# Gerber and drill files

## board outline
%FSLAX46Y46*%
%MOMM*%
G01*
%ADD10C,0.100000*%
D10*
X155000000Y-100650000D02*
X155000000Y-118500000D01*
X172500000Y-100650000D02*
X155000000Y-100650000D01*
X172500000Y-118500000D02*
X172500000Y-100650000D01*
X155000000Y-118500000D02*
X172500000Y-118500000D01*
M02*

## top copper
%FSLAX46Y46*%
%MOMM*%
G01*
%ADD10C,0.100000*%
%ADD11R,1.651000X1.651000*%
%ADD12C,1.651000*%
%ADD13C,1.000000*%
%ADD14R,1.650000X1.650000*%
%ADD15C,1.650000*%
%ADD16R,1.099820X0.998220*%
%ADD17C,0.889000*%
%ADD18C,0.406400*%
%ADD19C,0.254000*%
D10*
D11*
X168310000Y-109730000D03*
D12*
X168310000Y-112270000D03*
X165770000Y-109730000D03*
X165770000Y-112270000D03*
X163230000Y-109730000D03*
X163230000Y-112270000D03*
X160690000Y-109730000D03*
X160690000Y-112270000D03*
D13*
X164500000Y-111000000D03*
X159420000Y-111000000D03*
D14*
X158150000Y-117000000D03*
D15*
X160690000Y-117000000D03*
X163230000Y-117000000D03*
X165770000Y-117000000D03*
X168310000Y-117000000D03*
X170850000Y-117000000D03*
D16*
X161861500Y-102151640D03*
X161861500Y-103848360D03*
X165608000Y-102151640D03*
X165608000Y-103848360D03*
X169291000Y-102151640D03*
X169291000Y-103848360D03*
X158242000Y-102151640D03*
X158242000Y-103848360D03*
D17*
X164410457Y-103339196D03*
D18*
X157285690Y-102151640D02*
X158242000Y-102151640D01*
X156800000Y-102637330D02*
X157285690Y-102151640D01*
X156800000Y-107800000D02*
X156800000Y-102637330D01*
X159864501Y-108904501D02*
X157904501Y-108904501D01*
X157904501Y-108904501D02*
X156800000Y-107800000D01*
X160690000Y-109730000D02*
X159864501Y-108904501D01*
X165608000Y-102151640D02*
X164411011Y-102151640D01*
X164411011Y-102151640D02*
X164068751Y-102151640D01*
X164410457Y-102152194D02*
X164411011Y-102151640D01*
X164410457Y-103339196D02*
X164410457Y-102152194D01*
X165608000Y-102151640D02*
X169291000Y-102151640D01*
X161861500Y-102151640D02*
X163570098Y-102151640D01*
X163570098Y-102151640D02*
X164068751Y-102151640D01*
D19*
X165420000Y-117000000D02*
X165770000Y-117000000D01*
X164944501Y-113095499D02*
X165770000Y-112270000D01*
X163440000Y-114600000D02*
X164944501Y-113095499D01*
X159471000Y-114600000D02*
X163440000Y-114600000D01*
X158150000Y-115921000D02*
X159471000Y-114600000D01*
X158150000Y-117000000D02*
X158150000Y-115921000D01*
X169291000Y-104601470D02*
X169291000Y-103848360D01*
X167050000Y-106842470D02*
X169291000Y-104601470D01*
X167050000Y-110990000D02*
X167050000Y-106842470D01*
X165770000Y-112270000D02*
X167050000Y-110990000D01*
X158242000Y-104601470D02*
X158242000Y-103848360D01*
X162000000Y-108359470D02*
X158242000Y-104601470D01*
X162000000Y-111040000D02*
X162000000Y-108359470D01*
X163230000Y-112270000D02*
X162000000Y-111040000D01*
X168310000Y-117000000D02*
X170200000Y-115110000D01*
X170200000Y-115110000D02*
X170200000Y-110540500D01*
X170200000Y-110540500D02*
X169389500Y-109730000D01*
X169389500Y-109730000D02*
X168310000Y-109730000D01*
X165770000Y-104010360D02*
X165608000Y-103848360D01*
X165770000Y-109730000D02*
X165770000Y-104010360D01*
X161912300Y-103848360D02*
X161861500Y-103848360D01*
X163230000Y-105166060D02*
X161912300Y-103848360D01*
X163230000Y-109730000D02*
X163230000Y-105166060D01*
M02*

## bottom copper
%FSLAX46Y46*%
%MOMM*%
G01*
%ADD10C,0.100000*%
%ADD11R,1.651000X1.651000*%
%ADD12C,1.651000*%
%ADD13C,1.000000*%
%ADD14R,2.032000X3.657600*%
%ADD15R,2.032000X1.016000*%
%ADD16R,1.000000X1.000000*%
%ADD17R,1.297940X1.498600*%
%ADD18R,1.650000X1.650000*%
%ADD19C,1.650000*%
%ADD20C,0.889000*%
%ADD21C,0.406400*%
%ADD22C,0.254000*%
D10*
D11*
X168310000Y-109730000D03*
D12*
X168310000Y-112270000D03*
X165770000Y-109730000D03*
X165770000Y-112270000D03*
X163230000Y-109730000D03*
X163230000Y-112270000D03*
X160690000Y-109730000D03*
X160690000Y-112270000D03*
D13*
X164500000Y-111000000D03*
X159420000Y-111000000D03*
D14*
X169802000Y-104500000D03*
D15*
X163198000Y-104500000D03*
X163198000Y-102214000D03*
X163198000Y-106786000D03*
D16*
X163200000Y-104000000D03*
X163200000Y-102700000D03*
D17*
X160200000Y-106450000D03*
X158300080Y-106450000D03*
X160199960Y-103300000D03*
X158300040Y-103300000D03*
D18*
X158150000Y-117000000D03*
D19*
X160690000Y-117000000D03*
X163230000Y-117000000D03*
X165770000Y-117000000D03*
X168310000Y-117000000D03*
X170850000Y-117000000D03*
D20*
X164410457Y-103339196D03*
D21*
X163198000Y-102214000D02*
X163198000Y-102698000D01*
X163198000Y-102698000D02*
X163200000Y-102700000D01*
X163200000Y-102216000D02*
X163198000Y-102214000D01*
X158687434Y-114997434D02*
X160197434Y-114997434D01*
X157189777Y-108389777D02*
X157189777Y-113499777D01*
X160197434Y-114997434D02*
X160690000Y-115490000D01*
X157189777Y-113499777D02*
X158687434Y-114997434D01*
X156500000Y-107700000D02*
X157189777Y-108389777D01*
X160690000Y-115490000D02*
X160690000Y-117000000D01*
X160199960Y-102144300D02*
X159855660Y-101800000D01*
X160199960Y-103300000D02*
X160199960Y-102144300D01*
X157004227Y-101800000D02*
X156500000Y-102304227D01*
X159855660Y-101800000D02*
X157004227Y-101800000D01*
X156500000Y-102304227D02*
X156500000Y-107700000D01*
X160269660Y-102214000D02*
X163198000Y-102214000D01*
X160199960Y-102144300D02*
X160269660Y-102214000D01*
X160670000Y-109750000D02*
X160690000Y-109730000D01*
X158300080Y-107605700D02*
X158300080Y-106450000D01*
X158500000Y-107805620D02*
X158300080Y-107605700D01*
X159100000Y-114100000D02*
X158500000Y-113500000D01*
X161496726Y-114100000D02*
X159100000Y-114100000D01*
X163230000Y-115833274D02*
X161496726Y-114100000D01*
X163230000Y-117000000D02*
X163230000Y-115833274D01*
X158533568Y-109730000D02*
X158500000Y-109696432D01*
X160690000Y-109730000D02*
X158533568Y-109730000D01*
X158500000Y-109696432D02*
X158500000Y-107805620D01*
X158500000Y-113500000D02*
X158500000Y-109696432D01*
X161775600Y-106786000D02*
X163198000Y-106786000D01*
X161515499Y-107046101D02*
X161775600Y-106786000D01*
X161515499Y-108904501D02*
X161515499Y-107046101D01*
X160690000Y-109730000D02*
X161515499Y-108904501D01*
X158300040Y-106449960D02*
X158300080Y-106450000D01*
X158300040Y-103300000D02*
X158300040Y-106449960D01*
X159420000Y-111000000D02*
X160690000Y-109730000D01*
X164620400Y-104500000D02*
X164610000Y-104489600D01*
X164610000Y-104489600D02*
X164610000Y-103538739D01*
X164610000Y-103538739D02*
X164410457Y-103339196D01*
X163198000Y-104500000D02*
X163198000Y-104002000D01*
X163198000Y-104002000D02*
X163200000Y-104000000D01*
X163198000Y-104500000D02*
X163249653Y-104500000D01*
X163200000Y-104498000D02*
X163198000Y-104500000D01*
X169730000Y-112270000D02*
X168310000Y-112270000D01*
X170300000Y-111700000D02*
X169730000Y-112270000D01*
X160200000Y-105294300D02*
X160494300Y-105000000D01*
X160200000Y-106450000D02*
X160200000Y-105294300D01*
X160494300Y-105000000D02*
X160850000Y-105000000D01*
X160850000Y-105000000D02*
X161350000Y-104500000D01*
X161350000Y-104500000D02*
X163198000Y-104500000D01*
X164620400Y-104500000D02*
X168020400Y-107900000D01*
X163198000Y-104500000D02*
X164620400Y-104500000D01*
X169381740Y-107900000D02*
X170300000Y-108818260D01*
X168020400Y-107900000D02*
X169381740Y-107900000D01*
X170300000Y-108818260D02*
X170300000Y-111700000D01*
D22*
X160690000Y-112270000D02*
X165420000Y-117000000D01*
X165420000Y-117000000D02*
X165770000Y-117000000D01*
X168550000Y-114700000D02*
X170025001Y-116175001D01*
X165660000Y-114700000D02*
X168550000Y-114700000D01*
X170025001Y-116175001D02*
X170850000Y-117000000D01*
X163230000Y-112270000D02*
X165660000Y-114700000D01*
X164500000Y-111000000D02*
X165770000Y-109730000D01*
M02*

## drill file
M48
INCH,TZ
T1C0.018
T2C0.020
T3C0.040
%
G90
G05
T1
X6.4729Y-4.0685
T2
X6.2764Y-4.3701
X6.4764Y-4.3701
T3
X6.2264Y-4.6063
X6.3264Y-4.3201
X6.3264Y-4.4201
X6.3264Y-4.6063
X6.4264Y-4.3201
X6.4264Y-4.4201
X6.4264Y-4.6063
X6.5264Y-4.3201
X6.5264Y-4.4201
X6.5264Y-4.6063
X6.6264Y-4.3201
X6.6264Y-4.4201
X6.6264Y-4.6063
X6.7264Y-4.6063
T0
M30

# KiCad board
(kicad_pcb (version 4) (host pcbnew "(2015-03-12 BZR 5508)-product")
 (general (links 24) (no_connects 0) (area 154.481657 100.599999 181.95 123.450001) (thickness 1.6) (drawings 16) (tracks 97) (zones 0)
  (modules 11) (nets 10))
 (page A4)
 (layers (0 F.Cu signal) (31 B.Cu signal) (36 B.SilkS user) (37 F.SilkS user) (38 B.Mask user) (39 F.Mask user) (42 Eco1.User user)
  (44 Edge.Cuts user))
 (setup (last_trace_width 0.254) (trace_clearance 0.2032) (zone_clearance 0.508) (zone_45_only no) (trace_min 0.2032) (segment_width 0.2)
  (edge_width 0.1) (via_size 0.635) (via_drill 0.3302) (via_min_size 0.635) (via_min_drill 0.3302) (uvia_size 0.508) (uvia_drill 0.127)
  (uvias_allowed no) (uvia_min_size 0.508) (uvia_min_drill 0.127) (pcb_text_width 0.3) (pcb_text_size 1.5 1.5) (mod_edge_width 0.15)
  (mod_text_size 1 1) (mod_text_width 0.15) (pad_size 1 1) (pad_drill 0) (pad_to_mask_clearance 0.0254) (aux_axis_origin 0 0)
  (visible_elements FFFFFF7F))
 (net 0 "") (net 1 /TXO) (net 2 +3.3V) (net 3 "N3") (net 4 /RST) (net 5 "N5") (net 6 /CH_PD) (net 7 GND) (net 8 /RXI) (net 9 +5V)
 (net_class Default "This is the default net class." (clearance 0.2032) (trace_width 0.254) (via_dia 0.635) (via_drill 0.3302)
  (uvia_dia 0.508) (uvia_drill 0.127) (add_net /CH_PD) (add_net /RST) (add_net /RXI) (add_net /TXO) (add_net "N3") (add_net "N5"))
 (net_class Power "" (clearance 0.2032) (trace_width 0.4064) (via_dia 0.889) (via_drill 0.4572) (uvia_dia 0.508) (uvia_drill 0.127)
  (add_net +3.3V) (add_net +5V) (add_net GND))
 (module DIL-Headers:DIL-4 (layer F.Cu) (at 164.5 111)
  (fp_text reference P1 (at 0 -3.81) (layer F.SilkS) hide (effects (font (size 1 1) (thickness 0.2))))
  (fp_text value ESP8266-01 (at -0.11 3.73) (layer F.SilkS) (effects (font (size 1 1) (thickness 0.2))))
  (pad 1 thru_hole rect (at 3.81 -1.27) (size 1.651 1.651) (drill 1.016) (layers *.Cu *.Mask F.SilkS) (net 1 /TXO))
  (pad 2 thru_hole circle (at 3.81 1.27) (size 1.651 1.651) (drill 1.016) (layers *.Cu *.Mask F.SilkS) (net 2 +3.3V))
  (pad 3 thru_hole circle (at 1.27 -1.27) (size 1.651 1.651) (drill 1.016) (layers *.Cu *.Mask F.SilkS) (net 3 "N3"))
  (pad 4 thru_hole circle (at 1.27 1.27) (size 1.651 1.651) (drill 1.016) (layers *.Cu *.Mask F.SilkS) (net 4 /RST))
  (pad 5 thru_hole circle (at -1.27 -1.27) (size 1.651 1.651) (drill 1.016) (layers *.Cu *.Mask F.SilkS) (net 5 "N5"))
  (pad 6 thru_hole circle (at -1.27 1.27) (size 1.651 1.651) (drill 1.016) (layers *.Cu *.Mask F.SilkS) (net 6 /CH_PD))
  (pad 7 thru_hole circle (at -3.81 -1.27) (size 1.651 1.651) (drill 1.016) (layers *.Cu *.Mask F.SilkS) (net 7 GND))
  (pad 8 thru_hole circle (at -3.81 1.27) (size 1.651 1.651) (drill 1.016) (layers *.Cu *.Mask F.SilkS) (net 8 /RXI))
  (pad 3 thru_hole circle (at 0 0) (size 1 1) (drill 0.5) (layers *.Cu *.Mask F.SilkS) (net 3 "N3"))
  (pad 7 thru_hole circle (at -5.08 0) (size 1 1) (drill 0.5) (layers *.Cu *.Mask F.SilkS) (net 7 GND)))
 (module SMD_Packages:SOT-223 (layer B.Cu) (at 166.5 104.5 90)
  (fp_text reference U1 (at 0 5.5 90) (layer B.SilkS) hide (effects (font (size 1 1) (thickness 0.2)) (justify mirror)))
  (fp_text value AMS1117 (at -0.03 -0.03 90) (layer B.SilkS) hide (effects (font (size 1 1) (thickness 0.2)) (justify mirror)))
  (pad 4 smd rect (at 0 3.302 90) (size 3.6576 2.032) (layers B.Cu B.Mask))
  (pad 2 smd rect (at 0 -3.302 90) (size 1.016 2.032) (layers B.Cu B.Mask) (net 2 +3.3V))
  (pad 3 smd rect (at 2.286 -3.302 90) (size 1.016 2.032) (layers B.Cu B.Mask) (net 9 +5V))
  (pad 1 smd rect (at -2.286 -3.302 90) (size 1.016 2.032) (layers B.Cu B.Mask) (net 7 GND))
  (pad 2 smd rect (at 0.5 -3.3 90) (size 1 1) (layers B.Cu B.Mask) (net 2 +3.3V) (solder_mask_margin 0.15) (clearance 0.01))
  (pad 3 smd rect (at 1.8 -3.3 90) (size 1 1) (layers B.Cu B.Mask) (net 9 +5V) (solder_mask_margin 0.15) (clearance 0.01)))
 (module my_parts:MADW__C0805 (layer B.Cu) (at 159.25004 106.45 180)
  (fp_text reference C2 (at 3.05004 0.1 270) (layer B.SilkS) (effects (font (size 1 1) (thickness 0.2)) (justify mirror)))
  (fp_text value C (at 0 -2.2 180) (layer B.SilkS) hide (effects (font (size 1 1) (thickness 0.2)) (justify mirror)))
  (pad 1 smd rect (at -0.94996 0 180) (size 1.29794 1.4986) (layers B.Cu B.Mask) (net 2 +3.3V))
  (pad 2 smd rect (at 0.94996 0 180) (size 1.29794 1.4986) (layers B.Cu B.Mask) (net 7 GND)))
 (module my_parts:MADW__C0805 (layer B.Cu) (at 159.25 103.3 180)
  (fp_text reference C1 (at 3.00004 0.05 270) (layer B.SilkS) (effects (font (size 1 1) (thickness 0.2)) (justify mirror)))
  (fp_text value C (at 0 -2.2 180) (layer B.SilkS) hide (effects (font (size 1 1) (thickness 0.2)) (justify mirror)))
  (pad 1 smd rect (at -0.94996 0 180) (size 1.29794 1.4986) (layers B.Cu B.Mask) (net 9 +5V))
  (pad 2 smd rect (at 0.94996 0 180) (size 1.29794 1.4986) (layers B.Cu B.Mask) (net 7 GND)))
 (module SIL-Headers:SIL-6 (layer F.Cu) (at 164.5 117)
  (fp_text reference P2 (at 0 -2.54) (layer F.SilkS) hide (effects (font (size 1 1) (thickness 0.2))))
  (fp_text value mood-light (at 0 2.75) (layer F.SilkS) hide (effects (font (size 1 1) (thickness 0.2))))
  (pad 1 thru_hole rect (at -6.35 0) (size 1.65 1.65) (drill 1.016) (layers *.Cu *.Mask F.SilkS) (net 4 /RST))
  (pad 2 thru_hole circle (at -3.81 0) (size 1.65 1.65) (drill 1.016) (layers *.Cu *.Mask F.SilkS) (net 9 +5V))
  (pad 3 thru_hole circle (at -1.27 0) (size 1.65 1.65) (drill 1.016) (layers *.Cu *.Mask F.SilkS) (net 7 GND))
  (pad 4 thru_hole circle (at 1.27 0) (size 1.65 1.65) (drill 1.016) (layers *.Cu *.Mask F.SilkS) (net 8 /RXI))
  (pad 5 thru_hole circle (at 3.81 0) (size 1.65 1.65) (drill 1.016) (layers *.Cu *.Mask F.SilkS) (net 1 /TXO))
  (pad 6 thru_hole circle (at 6.35 0) (size 1.65 1.65) (drill 1.016) (layers *.Cu *.Mask F.SilkS) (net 6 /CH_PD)))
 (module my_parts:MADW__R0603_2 (layer F.Cu) (at 161.8615 103 270)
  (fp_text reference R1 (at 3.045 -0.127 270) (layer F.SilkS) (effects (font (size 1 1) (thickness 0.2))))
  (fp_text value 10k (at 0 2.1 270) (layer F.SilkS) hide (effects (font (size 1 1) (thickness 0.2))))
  (pad 1 smd rect (at -0.84836 0 270) (size 0.99822 1.09982) (layers F.Cu F.Mask) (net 2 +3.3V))
  (pad 2 smd rect (at 0.84836 0 270) (size 0.99822 1.09982) (layers F.Cu F.Mask) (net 5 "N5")))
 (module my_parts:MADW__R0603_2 (layer F.Cu) (at 165.608 103 270)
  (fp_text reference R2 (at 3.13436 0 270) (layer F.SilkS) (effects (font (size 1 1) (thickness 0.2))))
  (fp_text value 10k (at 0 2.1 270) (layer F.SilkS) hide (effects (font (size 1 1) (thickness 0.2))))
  (pad 1 smd rect (at -0.84836 0 270) (size 0.99822 1.09982) (layers F.Cu F.Mask) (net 2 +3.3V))
  (pad 2 smd rect (at 0.84836 0 270) (size 0.99822 1.09982) (layers F.Cu F.Mask) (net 3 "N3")))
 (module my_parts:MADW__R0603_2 (layer F.Cu) (at 169.291 103 270)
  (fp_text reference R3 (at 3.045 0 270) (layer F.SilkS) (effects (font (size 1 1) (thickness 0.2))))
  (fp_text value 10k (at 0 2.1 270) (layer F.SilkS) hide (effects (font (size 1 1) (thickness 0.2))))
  (pad 1 smd rect (at -0.84836 0 270) (size 0.99822 1.09982) (layers F.Cu F.Mask) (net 2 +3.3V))
  (pad 2 smd rect (at 0.84836 0 270) (size 0.99822 1.09982) (layers F.Cu F.Mask) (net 4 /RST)))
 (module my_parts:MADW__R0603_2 (layer F.Cu) (at 158.242 103 270)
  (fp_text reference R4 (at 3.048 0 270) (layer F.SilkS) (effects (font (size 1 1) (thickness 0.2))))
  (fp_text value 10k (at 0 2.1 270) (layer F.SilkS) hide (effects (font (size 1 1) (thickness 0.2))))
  (pad 1 smd rect (at -0.84836 0 270) (size 0.99822 1.09982) (layers F.Cu F.Mask) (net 7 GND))
  (pad 2 smd rect (at 0.84836 0 270) (size 0.99822 1.09982) (layers F.Cu F.Mask) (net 6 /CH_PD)))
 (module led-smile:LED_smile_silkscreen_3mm (layer F.Cu) (at 157.05 109.75)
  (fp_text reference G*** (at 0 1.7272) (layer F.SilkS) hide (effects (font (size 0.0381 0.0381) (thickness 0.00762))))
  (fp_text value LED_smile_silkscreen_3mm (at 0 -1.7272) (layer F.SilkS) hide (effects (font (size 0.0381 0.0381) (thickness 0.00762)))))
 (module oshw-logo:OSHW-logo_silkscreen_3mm (layer F.Cu) (at 157 113)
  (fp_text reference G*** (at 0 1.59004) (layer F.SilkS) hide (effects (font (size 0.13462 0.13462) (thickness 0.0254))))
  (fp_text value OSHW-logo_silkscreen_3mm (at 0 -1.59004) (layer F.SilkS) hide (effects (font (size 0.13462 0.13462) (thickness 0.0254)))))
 (gr_line (start 155 100.65) (end 155 118.5) (layer Edge.Cuts) (width 0.1))
 (gr_line (start 172.5 100.65) (end 155 100.65) (layer Edge.Cuts) (width 0.1))
 (gr_line (start 172.5 118.5) (end 172.5 100.65) (layer Edge.Cuts) (width 0.1))
 (gr_line (start 155 118.5) (end 172.5 118.5) (layer Edge.Cuts) (width 0.1))
 (segment (start 163.198 102.214) (end 163.198 102.698) (width 0.4064) (layer B.Cu) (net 9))
 (segment (start 163.198 102.698) (end 163.2 102.7) (width 0.4064) (layer B.Cu) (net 9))
 (segment (start 163.2 102.216) (end 163.198 102.214) (width 0.4064) (layer B.Cu) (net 9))
 (segment (start 158.687434 114.997434) (end 160.197434 114.997434) (width 0.4064) (layer B.Cu) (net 9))
 (segment (start 157.189777 108.389777) (end 157.189777 113.499777) (width 0.4064) (layer B.Cu) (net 9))
 (segment (start 160.197434 114.997434) (end 160.69 115.49) (width 0.4064) (layer B.Cu) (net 9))
 (segment (start 157.189777 113.499777) (end 158.687434 114.997434) (width 0.4064) (layer B.Cu) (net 9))
 (segment (start 156.5 107.7) (end 157.189777 108.389777) (width 0.4064) (layer B.Cu) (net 9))
 (segment (start 160.69 115.49) (end 160.69 117) (width 0.4064) (layer B.Cu) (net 9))
 (segment (start 160.19996 102.1443) (end 159.85566 101.8) (width 0.4064) (layer B.Cu) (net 9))
 (segment (start 160.19996 103.3) (end 160.19996 102.1443) (width 0.4064) (layer B.Cu) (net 9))
 (segment (start 157.004227 101.8) (end 156.5 102.304227) (width 0.4064) (layer B.Cu) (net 9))
 (segment (start 159.85566 101.8) (end 157.004227 101.8) (width 0.4064) (layer B.Cu) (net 9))
 (segment (start 156.5 102.304227) (end 156.5 107.7) (width 0.4064) (layer B.Cu) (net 9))
 (segment (start 160.26966 102.214) (end 163.198 102.214) (width 0.4064) (layer B.Cu) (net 9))
 (segment (start 160.19996 102.1443) (end 160.26966 102.214) (width 0.4064) (layer B.Cu) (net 9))
 (segment (start 160.67 109.75) (end 160.69 109.73) (width 0.4064) (layer B.Cu) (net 7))
 (segment (start 158.30008 107.6057) (end 158.30008 106.45) (width 0.4064) (layer B.Cu) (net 7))
 (segment (start 158.5 107.80562) (end 158.30008 107.6057) (width 0.4064) (layer B.Cu) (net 7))
 (segment (start 159.1 114.1) (end 158.5 113.5) (width 0.4064) (layer B.Cu) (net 7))
 (segment (start 161.496726 114.1) (end 159.1 114.1) (width 0.4064) (layer B.Cu) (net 7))
 (segment (start 163.23 115.833274) (end 161.496726 114.1) (width 0.4064) (layer B.Cu) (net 7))
 (segment (start 163.23 117) (end 163.23 115.833274) (width 0.4064) (layer B.Cu) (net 7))
 (segment (start 158.533568 109.73) (end 158.5 109.696432) (width 0.4064) (layer B.Cu) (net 7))
 (segment (start 160.69 109.73) (end 158.533568 109.73) (width 0.4064) (layer B.Cu) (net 7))
 (segment (start 158.5 109.696432) (end 158.5 107.80562) (width 0.4064) (layer B.Cu) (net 7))
 (segment (start 158.5 113.5) (end 158.5 109.696432) (width 0.4064) (layer B.Cu) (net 7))
 (segment (start 161.7756 106.786) (end 163.198 106.786) (width 0.4064) (layer B.Cu) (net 7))
 (segment (start 161.515499 107.046101) (end 161.7756 106.786) (width 0.4064) (layer B.Cu) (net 7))
 (segment (start 161.515499 108.904501) (end 161.515499 107.046101) (width 0.4064) (layer B.Cu) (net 7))
 (segment (start 160.69 109.73) (end 161.515499 108.904501) (width 0.4064) (layer B.Cu) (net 7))
 (segment (start 157.28569 102.15164) (end 158.242 102.15164) (width 0.4064) (layer F.Cu) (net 7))
 (segment (start 156.8 102.63733) (end 157.28569 102.15164) (width 0.4064) (layer F.Cu) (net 7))
 (segment (start 156.8 107.8) (end 156.8 102.63733) (width 0.4064) (layer F.Cu) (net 7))
 (segment (start 159.864501 108.904501) (end 157.904501 108.904501) (width 0.4064) (layer F.Cu) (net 7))
 (segment (start 157.904501 108.904501) (end 156.8 107.8) (width 0.4064) (layer F.Cu) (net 7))
 (segment (start 160.69 109.73) (end 159.864501 108.904501) (width 0.4064) (layer F.Cu) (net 7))
 (segment (start 158.30004 106.44996) (end 158.30008 106.45) (width 0.4064) (layer B.Cu) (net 7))
 (segment (start 158.30004 103.3) (end 158.30004 106.44996) (width 0.4064) (layer B.Cu) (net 7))
 (segment (start 159.42 111) (end 160.69 109.73) (width 0.4064) (layer B.Cu) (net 7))
 (segment (start 164.6204 104.5) (end 164.61 104.4896) (width 0.4064) (layer B.Cu) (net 2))
 (segment (start 164.61 104.4896) (end 164.61 103.538739) (width 0.4064) (layer B.Cu) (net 2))
 (segment (start 164.61 103.538739) (end 164.410457 103.339196) (width 0.4064) (layer B.Cu) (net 2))
 (segment (start 165.608 102.15164) (end 164.411011 102.15164) (width 0.4064) (layer F.Cu) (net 2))
 (segment (start 164.411011 102.15164) (end 164.068751 102.15164) (width 0.4064) (layer F.Cu) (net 2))
 (segment (start 164.410457 102.152194) (end 164.411011 102.15164) (width 0.4064) (layer F.Cu) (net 2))
 (segment (start 164.410457 103.339196) (end 164.410457 102.152194) (width 0.4064) (layer F.Cu) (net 2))
 (segment (start 163.198 104.5) (end 163.198 104.002) (width 0.4064) (layer B.Cu) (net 2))
 (segment (start 163.198 104.002) (end 163.2 104) (width 0.4064) (layer B.Cu) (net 2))
 (segment (start 163.198 104.5) (end 163.249653 104.5) (width 0.4064) (layer B.Cu) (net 2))
 (via (at 164.410457 103.339196) (size 0.889) (drill 0.4572) (layers F.Cu B.Cu) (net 2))
 (segment (start 163.2 104.498) (end 163.198 104.5) (width 0.4064) (layer B.Cu) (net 2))
 (segment (start 169.73 112.27) (end 168.31 112.27) (width 0.4064) (layer B.Cu) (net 2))
 (segment (start 170.3 111.7) (end 169.73 112.27) (width 0.4064) (layer B.Cu) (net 2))
 (segment (start 165.608 102.15164) (end 169.291 102.15164) (width 0.4064) (layer F.Cu) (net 2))
 (segment (start 160.2 105.2943) (end 160.4943 105) (width 0.4064) (layer B.Cu) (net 2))
 (segment (start 160.2 106.45) (end 160.2 105.2943) (width 0.4064) (layer B.Cu) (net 2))
 (segment (start 160.4943 105) (end 160.85 105) (width 0.4064) (layer B.Cu) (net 2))
 (segment (start 160.85 105) (end 161.35 104.5) (width 0.4064) (layer B.Cu) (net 2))
 (segment (start 161.35 104.5) (end 163.198 104.5) (width 0.4064) (layer B.Cu) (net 2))
 (segment (start 164.6204 104.5) (end 168.0204 107.9) (width 0.4064) (layer B.Cu) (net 2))
 (segment (start 163.198 104.5) (end 164.6204 104.5) (width 0.4064) (layer B.Cu) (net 2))
 (segment (start 169.38174 107.9) (end 170.3 108.81826) (width 0.4064) (layer B.Cu) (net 2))
 (segment (start 168.0204 107.9) (end 169.38174 107.9) (width 0.4064) (layer B.Cu) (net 2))
 (segment (start 170.3 108.81826) (end 170.3 111.7) (width 0.4064) (layer B.Cu) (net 2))
 (segment (start 161.8615 102.15164) (end 163.570098 102.15164) (width 0.4064) (layer F.Cu) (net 2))
 (segment (start 163.570098 102.15164) (end 164.068751 102.15164) (width 0.4064) (layer F.Cu) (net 2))
 (segment (start 160.69 112.27) (end 165.42 117) (width 0.254) (layer B.Cu) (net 8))
 (segment (start 165.42 117) (end 165.77 117) (width 0.254) (layer F.Cu) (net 8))
 (segment (start 165.42 117) (end 165.77 117) (width 0.254) (layer B.Cu) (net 8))
 (segment (start 164.944501 113.095499) (end 165.77 112.27) (width 0.254) (layer F.Cu) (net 4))
 (segment (start 163.44 114.6) (end 164.944501 113.095499) (width 0.254) (layer F.Cu) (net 4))
 (segment (start 159.471 114.6) (end 163.44 114.6) (width 0.254) (layer F.Cu) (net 4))
 (segment (start 158.15 115.921) (end 159.471 114.6) (width 0.254) (layer F.Cu) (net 4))
 (segment (start 158.15 117) (end 158.15 115.921) (width 0.254) (layer F.Cu) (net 4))
 (segment (start 169.291 104.60147) (end 169.291 103.84836) (width 0.254) (layer F.Cu) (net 4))
 (segment (start 167.05 106.84247) (end 169.291 104.60147) (width 0.254) (layer F.Cu) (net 4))
 (segment (start 167.05 110.99) (end 167.05 106.84247) (width 0.254) (layer F.Cu) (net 4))
 (segment (start 165.77 112.27) (end 167.05 110.99) (width 0.254) (layer F.Cu) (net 4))
 (segment (start 168.55 114.7) (end 170.025001 116.175001) (width 0.254) (layer B.Cu) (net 6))
 (segment (start 165.66 114.7) (end 168.55 114.7) (width 0.254) (layer B.Cu) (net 6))
 (segment (start 170.025001 116.175001) (end 170.85 117) (width 0.254) (layer B.Cu) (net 6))
 (segment (start 163.23 112.27) (end 165.66 114.7) (width 0.254) (layer B.Cu) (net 6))
 (segment (start 158.242 104.60147) (end 158.242 103.84836) (width 0.254) (layer F.Cu) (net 6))
 (segment (start 162 108.35947) (end 158.242 104.60147) (width 0.254) (layer F.Cu) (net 6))
 (segment (start 162 111.04) (end 162 108.35947) (width 0.254) (layer F.Cu) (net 6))
 (segment (start 163.23 112.27) (end 162 111.04) (width 0.254) (layer F.Cu) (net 6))
 (segment (start 168.31 117) (end 170.2 115.11) (width 0.254) (layer F.Cu) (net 1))
 (segment (start 170.2 115.11) (end 170.2 110.5405) (width 0.254) (layer F.Cu) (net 1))
 (segment (start 170.2 110.5405) (end 169.3895 109.73) (width 0.254) (layer F.Cu) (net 1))
 (segment (start 169.3895 109.73) (end 168.31 109.73) (width 0.254) (layer F.Cu) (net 1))
 (segment (start 165.77 104.01036) (end 165.608 103.84836) (width 0.254) (layer F.Cu) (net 3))
 (segment (start 165.77 109.73) (end 165.77 104.01036) (width 0.254) (layer F.Cu) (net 3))
 (segment (start 164.5 111) (end 165.77 109.73) (width 0.254) (layer B.Cu) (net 3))
 (segment (start 161.9123 103.84836) (end 161.8615 103.84836) (width 0.254) (layer F.Cu) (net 5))
 (segment (start 163.23 105.16606) (end 161.9123 103.84836) (width 0.254) (layer F.Cu) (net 5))
 (segment (start 163.23 109.73) (end 163.23 105.16606) (width 0.254) (layer F.Cu) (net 5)))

